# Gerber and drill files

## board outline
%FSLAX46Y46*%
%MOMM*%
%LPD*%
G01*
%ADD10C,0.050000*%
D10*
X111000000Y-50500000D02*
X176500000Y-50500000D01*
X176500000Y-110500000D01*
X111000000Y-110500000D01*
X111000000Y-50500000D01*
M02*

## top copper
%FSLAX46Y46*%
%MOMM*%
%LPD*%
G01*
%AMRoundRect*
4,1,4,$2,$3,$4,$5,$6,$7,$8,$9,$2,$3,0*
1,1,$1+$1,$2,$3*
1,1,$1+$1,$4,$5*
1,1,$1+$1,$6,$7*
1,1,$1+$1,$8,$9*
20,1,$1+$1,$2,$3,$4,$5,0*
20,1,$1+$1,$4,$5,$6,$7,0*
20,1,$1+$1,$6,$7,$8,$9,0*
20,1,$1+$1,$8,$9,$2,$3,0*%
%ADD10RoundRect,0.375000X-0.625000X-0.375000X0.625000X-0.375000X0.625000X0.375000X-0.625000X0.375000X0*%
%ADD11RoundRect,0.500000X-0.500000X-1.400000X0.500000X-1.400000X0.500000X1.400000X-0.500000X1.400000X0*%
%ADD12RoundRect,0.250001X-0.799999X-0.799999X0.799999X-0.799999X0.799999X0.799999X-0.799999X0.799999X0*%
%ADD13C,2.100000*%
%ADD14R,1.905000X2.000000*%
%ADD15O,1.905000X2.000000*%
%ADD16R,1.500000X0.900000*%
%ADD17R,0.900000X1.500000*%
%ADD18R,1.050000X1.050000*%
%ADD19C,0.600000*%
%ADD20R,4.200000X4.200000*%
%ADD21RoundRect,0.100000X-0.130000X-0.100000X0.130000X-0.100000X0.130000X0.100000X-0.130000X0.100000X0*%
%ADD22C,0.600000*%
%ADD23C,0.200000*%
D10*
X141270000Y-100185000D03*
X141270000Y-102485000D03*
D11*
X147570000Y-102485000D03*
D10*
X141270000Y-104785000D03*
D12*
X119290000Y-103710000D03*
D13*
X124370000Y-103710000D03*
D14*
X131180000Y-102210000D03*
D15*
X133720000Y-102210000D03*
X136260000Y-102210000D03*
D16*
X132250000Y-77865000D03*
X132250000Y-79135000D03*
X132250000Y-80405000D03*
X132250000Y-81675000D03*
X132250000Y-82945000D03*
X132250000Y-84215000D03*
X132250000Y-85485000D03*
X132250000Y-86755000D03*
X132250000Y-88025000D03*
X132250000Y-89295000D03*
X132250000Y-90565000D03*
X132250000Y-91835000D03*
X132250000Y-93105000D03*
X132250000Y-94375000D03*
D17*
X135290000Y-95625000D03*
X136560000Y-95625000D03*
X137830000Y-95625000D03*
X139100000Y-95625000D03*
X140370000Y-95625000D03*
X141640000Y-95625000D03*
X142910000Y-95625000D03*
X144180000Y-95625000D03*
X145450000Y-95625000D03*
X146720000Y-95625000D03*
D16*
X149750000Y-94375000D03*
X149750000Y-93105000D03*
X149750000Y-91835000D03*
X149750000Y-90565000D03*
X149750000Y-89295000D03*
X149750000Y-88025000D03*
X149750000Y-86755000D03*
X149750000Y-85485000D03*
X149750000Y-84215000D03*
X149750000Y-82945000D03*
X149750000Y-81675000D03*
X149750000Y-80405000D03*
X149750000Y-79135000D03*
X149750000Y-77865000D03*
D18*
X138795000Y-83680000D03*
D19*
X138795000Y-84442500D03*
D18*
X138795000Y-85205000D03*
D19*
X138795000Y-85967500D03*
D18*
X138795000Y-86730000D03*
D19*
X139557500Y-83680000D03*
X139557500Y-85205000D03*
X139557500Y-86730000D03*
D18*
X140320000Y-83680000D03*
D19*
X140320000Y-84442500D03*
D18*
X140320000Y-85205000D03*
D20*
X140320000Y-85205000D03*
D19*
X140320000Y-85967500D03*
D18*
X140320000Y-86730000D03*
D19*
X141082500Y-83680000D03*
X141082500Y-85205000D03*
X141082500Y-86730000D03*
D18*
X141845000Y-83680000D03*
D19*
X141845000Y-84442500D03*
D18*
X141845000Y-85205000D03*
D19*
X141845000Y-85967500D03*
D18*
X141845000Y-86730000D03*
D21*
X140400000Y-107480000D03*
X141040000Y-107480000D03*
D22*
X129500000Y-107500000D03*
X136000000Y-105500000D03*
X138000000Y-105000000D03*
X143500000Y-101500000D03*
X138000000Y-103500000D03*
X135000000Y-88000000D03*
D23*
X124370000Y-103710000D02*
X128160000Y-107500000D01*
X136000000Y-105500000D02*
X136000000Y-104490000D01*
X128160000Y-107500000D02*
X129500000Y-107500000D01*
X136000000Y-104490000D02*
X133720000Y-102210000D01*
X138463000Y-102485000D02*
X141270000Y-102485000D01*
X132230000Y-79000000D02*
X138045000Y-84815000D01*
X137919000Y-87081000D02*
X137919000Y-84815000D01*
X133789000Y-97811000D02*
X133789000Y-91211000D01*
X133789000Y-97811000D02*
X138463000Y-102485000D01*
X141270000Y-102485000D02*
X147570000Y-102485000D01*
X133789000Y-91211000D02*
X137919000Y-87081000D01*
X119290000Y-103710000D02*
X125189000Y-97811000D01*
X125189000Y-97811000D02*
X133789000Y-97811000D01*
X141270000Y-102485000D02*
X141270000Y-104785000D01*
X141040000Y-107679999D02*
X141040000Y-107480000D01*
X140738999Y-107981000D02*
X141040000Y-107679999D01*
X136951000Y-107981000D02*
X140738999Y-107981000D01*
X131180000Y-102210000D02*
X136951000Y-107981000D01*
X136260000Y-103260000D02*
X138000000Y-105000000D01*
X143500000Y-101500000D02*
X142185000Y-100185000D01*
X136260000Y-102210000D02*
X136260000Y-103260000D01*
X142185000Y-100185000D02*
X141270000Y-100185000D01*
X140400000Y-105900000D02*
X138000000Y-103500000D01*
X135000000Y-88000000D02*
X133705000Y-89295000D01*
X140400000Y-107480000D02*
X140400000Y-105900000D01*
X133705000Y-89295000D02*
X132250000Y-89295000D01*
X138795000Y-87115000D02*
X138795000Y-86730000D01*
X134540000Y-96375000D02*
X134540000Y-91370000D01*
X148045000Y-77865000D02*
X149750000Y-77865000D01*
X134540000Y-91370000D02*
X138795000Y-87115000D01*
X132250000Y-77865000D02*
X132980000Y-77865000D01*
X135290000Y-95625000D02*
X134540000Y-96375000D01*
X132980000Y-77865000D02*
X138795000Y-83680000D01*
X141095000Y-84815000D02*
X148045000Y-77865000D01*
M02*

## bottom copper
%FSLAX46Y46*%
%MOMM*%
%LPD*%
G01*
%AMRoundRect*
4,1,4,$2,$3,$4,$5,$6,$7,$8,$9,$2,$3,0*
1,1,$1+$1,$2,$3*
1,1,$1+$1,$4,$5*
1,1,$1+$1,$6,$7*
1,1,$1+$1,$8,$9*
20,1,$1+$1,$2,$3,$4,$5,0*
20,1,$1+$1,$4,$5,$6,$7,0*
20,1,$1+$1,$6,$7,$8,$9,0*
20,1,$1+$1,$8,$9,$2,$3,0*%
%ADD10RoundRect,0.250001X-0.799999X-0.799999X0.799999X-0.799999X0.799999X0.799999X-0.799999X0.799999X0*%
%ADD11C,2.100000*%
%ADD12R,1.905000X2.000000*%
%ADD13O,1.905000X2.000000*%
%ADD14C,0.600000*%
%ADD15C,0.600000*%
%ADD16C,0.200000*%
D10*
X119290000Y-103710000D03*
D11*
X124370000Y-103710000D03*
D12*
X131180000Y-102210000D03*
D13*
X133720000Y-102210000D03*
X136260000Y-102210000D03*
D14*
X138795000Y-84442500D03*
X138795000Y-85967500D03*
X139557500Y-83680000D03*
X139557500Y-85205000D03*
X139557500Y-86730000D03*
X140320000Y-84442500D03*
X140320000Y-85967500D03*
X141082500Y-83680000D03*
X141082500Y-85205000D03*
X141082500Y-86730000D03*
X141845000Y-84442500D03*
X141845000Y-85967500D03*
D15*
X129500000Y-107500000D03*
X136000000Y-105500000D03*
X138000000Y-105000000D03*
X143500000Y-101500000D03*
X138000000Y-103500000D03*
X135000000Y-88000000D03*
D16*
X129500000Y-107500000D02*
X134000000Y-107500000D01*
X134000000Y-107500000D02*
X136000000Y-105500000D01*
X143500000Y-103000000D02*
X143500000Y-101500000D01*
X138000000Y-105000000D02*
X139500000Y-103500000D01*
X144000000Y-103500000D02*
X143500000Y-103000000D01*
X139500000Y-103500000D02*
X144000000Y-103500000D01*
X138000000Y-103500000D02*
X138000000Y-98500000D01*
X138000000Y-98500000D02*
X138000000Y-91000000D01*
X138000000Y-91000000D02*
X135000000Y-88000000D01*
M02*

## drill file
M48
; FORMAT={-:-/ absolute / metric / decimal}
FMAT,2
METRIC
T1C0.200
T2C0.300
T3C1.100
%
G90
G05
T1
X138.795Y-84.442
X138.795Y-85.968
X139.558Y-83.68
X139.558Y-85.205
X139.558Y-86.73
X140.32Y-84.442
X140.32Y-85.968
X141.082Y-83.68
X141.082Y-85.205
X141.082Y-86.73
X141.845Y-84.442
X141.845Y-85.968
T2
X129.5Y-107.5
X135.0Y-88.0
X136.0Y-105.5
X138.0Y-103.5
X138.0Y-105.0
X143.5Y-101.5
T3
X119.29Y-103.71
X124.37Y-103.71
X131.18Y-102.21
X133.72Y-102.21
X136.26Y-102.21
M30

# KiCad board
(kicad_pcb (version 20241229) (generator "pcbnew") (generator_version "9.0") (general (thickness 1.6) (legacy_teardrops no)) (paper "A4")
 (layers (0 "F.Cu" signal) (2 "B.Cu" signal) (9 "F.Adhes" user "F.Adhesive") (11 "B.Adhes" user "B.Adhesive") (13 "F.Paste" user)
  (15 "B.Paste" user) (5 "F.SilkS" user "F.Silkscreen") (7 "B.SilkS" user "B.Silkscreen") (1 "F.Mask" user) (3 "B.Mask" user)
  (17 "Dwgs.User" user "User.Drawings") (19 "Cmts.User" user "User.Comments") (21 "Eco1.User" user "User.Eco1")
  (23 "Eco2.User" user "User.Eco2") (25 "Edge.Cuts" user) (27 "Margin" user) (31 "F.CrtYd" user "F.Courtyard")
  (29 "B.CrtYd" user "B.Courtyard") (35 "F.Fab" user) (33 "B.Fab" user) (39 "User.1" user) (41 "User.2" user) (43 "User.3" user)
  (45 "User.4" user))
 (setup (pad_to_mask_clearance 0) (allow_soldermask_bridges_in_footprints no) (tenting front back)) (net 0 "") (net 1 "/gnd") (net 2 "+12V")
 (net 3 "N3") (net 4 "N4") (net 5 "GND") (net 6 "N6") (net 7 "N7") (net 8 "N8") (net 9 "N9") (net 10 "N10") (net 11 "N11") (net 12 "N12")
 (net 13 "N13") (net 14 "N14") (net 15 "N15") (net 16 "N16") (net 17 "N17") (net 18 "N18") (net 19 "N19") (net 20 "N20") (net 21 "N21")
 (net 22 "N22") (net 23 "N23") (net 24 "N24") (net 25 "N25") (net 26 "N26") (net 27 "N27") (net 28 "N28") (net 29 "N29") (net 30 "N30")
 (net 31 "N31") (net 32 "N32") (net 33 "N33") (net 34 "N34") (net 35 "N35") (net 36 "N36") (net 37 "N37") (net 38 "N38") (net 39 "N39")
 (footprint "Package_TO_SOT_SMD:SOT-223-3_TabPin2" (layer "F.Cu") (at 144.42 102.485)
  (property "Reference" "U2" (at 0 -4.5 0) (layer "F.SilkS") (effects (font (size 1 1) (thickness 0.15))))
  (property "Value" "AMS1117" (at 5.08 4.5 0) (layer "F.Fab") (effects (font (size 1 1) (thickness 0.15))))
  (pad "1" smd roundrect (at -3.15 -2.3) (size 2 1.5) (layers "F.Cu" "F.Mask" "F.Paste") (roundrect_rratio 0.25) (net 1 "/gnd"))
  (pad "2" smd roundrect (at -3.15 0) (size 2 1.5) (layers "F.Cu" "F.Mask" "F.Paste") (roundrect_rratio 0.25) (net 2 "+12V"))
  (pad "2" smd roundrect (at 3.15 0) (size 2 3.8) (layers "F.Cu" "F.Mask" "F.Paste") (roundrect_rratio 0.25) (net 2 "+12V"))
  (pad "3" smd roundrect (at -3.15 2.3) (size 2 1.5) (layers "F.Cu" "F.Mask" "F.Paste") (roundrect_rratio 0.25) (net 2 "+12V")))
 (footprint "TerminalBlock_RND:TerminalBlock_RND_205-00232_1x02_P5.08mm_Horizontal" (layer "F.Cu") (at 119.29 103.71)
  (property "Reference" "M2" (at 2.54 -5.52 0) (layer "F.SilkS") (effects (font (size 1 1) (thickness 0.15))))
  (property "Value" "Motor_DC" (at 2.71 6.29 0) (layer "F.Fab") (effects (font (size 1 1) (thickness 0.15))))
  (pad "1" thru_hole roundrect (at 0 0) (size 2.1 2.1) (drill 1.1) (layers "*.Cu" "*.Mask") (remove_unused_layers no)
   (roundrect_rratio 0.119048) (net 2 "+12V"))
  (pad "2" thru_hole circle (at 5.08 0) (size 2.1 2.1) (drill 1.1) (layers "*.Cu" "*.Mask") (remove_unused_layers no) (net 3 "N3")))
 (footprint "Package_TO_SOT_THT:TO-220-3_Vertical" (layer "F.Cu") (at 131.18 102.21)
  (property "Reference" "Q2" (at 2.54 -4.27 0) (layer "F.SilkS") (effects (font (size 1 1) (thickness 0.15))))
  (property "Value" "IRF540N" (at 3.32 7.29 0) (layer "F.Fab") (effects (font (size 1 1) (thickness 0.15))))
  (pad "1" thru_hole rect (at 0 0) (size 1.905 2) (drill 1.1) (layers "*.Cu" "*.Mask") (remove_unused_layers no) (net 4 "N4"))
  (pad "2" thru_hole oval (at 2.54 0) (size 1.905 2) (drill 1.1) (layers "*.Cu" "*.Mask") (remove_unused_layers no) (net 3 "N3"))
  (pad "3" thru_hole oval (at 5.08 0) (size 1.905 2) (drill 1.1) (layers "*.Cu" "*.Mask") (remove_unused_layers no) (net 1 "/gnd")))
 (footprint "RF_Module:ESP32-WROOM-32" (layer "F.Cu") (at 141 86.115)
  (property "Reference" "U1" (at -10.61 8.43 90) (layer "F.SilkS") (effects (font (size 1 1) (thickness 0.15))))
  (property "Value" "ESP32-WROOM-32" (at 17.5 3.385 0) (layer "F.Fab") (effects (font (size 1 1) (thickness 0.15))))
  (pad "1" smd rect (at -8.75 -8.25) (size 1.5 0.9) (layers "F.Cu" "F.Mask" "F.Paste") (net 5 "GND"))
  (pad "2" smd rect (at -8.75 -6.98) (size 1.5 0.9) (layers "F.Cu" "F.Mask" "F.Paste") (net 2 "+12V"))
  (pad "3" smd rect (at -8.75 -5.71) (size 1.5 0.9) (layers "F.Cu" "F.Mask" "F.Paste") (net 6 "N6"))
  (pad "4" smd rect (at -8.75 -4.44) (size 1.5 0.9) (layers "F.Cu" "F.Mask" "F.Paste") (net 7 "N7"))
  (pad "5" smd rect (at -8.75 -3.17) (size 1.5 0.9) (layers "F.Cu" "F.Mask" "F.Paste") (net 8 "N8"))
  (pad "6" smd rect (at -8.75 -1.9) (size 1.5 0.9) (layers "F.Cu" "F.Mask" "F.Paste") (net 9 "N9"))
  (pad "7" smd rect (at -8.75 -0.63) (size 1.5 0.9) (layers "F.Cu" "F.Mask" "F.Paste") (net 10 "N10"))
  (pad "8" smd rect (at -8.75 0.64) (size 1.5 0.9) (layers "F.Cu" "F.Mask" "F.Paste") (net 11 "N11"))
  (pad "9" smd rect (at -8.75 1.91) (size 1.5 0.9) (layers "F.Cu" "F.Mask" "F.Paste") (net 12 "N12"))
  (pad "10" smd rect (at -8.75 3.18) (size 1.5 0.9) (layers "F.Cu" "F.Mask" "F.Paste") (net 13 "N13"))
  (pad "11" smd rect (at -8.75 4.45) (size 1.5 0.9) (layers "F.Cu" "F.Mask" "F.Paste") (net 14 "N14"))
  (pad "12" smd rect (at -8.75 5.72) (size 1.5 0.9) (layers "F.Cu" "F.Mask" "F.Paste") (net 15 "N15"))
  (pad "13" smd rect (at -8.75 6.99) (size 1.5 0.9) (layers "F.Cu" "F.Mask" "F.Paste") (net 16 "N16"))
  (pad "14" smd rect (at -8.75 8.26) (size 1.5 0.9) (layers "F.Cu" "F.Mask" "F.Paste") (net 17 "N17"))
  (pad "15" smd rect (at -5.71 9.51 90) (size 1.5 0.9) (layers "F.Cu" "F.Mask" "F.Paste") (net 5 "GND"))
  (pad "16" smd rect (at -4.44 9.51 90) (size 1.5 0.9) (layers "F.Cu" "F.Mask" "F.Paste") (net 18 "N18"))
  (pad "17" smd rect (at -3.17 9.51 90) (size 1.5 0.9) (layers "F.Cu" "F.Mask" "F.Paste") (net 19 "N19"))
  (pad "18" smd rect (at -1.9 9.51 90) (size 1.5 0.9) (layers "F.Cu" "F.Mask" "F.Paste") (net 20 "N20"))
  (pad "19" smd rect (at -0.63 9.51 90) (size 1.5 0.9) (layers "F.Cu" "F.Mask" "F.Paste") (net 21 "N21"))
  (pad "20" smd rect (at 0.64 9.51 90) (size 1.5 0.9) (layers "F.Cu" "F.Mask" "F.Paste") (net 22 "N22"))
  (pad "21" smd rect (at 1.91 9.51 90) (size 1.5 0.9) (layers "F.Cu" "F.Mask" "F.Paste") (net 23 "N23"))
  (pad "22" smd rect (at 3.18 9.51 90) (size 1.5 0.9) (layers "F.Cu" "F.Mask" "F.Paste") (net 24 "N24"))
  (pad "23" smd rect (at 4.45 9.51 90) (size 1.5 0.9) (layers "F.Cu" "F.Mask" "F.Paste") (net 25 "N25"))
  (pad "24" smd rect (at 5.72 9.51 90) (size 1.5 0.9) (layers "F.Cu" "F.Mask" "F.Paste") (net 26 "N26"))
  (pad "25" smd rect (at 8.75 8.26) (size 1.5 0.9) (layers "F.Cu" "F.Mask" "F.Paste") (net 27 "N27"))
  (pad "26" smd rect (at 8.75 6.99) (size 1.5 0.9) (layers "F.Cu" "F.Mask" "F.Paste") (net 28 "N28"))
  (pad "27" smd rect (at 8.75 5.72) (size 1.5 0.9) (layers "F.Cu" "F.Mask" "F.Paste") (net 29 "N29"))
  (pad "28" smd rect (at 8.75 4.45) (size 1.5 0.9) (layers "F.Cu" "F.Mask" "F.Paste") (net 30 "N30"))
  (pad "29" smd rect (at 8.75 3.18) (size 1.5 0.9) (layers "F.Cu" "F.Mask" "F.Paste") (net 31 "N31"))
  (pad "30" smd rect (at 8.75 1.91) (size 1.5 0.9) (layers "F.Cu" "F.Mask" "F.Paste") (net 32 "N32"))
  (pad "31" smd rect (at 8.75 0.64) (size 1.5 0.9) (layers "F.Cu" "F.Mask" "F.Paste") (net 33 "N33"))
  (pad "32" smd rect (at 8.75 -0.63) (size 1.5 0.9) (layers "F.Cu" "F.Mask" "F.Paste") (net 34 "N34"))
  (pad "33" smd rect (at 8.75 -1.9) (size 1.5 0.9) (layers "F.Cu" "F.Mask" "F.Paste") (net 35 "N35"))
  (pad "34" smd rect (at 8.75 -3.17) (size 1.5 0.9) (layers "F.Cu" "F.Mask" "F.Paste") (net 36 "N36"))
  (pad "35" smd rect (at 8.75 -4.44) (size 1.5 0.9) (layers "F.Cu" "F.Mask" "F.Paste") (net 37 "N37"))
  (pad "36" smd rect (at 8.75 -5.71) (size 1.5 0.9) (layers "F.Cu" "F.Mask" "F.Paste") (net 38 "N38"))
  (pad "37" smd rect (at 8.75 -6.98) (size 1.5 0.9) (layers "F.Cu" "F.Mask" "F.Paste") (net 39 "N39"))
  (pad "38" smd rect (at 8.75 -8.25) (size 1.5 0.9) (layers "F.Cu" "F.Mask" "F.Paste") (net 5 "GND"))
  (pad "39" smd rect (at -2.205 -2.435) (size 1.05 1.05) (layers "F.Cu" "F.Paste") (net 5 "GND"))
  (pad "39" thru_hole circle (at -2.205 -1.6725) (size 0.6 0.6) (drill 0.2) (layers "*.Cu" "F.Mask") (remove_unused_layers no) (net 5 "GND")
   (zone_connect 2))
  (pad "39" smd rect (at -2.205 -0.91) (size 1.05 1.05) (layers "F.Cu" "F.Paste") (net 5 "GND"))
  (pad "39" thru_hole circle (at -2.205 -0.1475) (size 0.6 0.6) (drill 0.2) (layers "*.Cu" "F.Mask") (remove_unused_layers no) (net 5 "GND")
   (zone_connect 2))
  (pad "39" smd rect (at -2.205 0.615) (size 1.05 1.05) (layers "F.Cu" "F.Paste") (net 5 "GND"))
  (pad "39" thru_hole circle (at -1.4425 -2.435) (size 0.6 0.6) (drill 0.2) (layers "*.Cu" "F.Mask") (remove_unused_layers no) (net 5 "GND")
   (zone_connect 2))
  (pad "39" thru_hole circle (at -1.4425 -0.91) (size 0.6 0.6) (drill 0.2) (layers "*.Cu" "F.Mask") (remove_unused_layers no) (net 5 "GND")
   (zone_connect 2))
  (pad "39" thru_hole circle (at -1.4425 0.615) (size 0.6 0.6) (drill 0.2) (layers "*.Cu" "F.Mask") (remove_unused_layers no) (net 5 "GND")
   (zone_connect 2))
  (pad "39" smd rect (at -0.68 -2.435) (size 1.05 1.05) (layers "F.Cu" "F.Paste") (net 5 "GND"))
  (pad "39" thru_hole circle (at -0.68 -1.6725) (size 0.6 0.6) (drill 0.2) (layers "*.Cu" "F.Mask") (remove_unused_layers no) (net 5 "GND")
   (zone_connect 2))
  (pad "39" smd rect (at -0.68 -0.91) (size 1.05 1.05) (layers "F.Cu" "F.Paste") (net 5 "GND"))
  (pad "39" smd rect (at -0.68 -0.91) (size 4.2 4.2) (layers "F.Cu" "F.Mask") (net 5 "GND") (zone_connect 2))
  (pad "39" thru_hole circle (at -0.68 -0.1475) (size 0.6 0.6) (drill 0.2) (layers "*.Cu" "F.Mask") (remove_unused_layers no) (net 5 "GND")
   (zone_connect 2))
  (pad "39" smd rect (at -0.68 0.615) (size 1.05 1.05) (layers "F.Cu" "F.Paste") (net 5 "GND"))
  (pad "39" thru_hole circle (at 0.0825 -2.435) (size 0.6 0.6) (drill 0.2) (layers "*.Cu" "F.Mask") (remove_unused_layers no) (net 5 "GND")
   (zone_connect 2))
  (pad "39" thru_hole circle (at 0.0825 -0.91) (size 0.6 0.6) (drill 0.2) (layers "*.Cu" "F.Mask") (remove_unused_layers no) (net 5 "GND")
   (zone_connect 2))
  (pad "39" thru_hole circle (at 0.0825 0.615) (size 0.6 0.6) (drill 0.2) (layers "*.Cu" "F.Mask") (remove_unused_layers no) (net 5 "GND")
   (zone_connect 2))
  (pad "39" smd rect (at 0.845 -2.435) (size 1.05 1.05) (layers "F.Cu" "F.Paste") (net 5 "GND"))
  (pad "39" thru_hole circle (at 0.845 -1.6725) (size 0.6 0.6) (drill 0.2) (layers "*.Cu" "F.Mask") (remove_unused_layers no) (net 5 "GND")
   (zone_connect 2))
  (pad "39" smd rect (at 0.845 -0.91) (size 1.05 1.05) (layers "F.Cu" "F.Paste") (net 5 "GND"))
  (pad "39" thru_hole circle (at 0.845 -0.1475) (size 0.6 0.6) (drill 0.2) (layers "*.Cu" "F.Mask") (remove_unused_layers no) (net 5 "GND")
   (zone_connect 2))
  (pad "39" smd rect (at 0.845 0.615) (size 1.05 1.05) (layers "F.Cu" "F.Paste") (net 5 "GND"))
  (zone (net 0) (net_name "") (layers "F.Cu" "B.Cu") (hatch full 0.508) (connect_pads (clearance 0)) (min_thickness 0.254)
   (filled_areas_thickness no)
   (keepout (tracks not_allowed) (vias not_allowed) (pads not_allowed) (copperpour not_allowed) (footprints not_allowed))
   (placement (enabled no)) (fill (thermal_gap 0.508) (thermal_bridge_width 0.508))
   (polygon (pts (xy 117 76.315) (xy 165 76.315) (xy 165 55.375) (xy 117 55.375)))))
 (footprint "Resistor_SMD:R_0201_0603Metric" (layer "F.Cu") (at 140.72 107.48)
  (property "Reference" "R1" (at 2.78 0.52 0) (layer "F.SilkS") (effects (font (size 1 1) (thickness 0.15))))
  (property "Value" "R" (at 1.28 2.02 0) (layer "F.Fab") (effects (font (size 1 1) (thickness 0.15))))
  (pad "" smd roundrect (at -0.345 0) (size 0.318 0.36) (layers "F.Paste") (roundrect_rratio 0.25))
  (pad "" smd roundrect (at 0.345 0) (size 0.318 0.36) (layers "F.Paste") (roundrect_rratio 0.25))
  (pad "1" smd roundrect (at -0.32 0) (size 0.46 0.4) (layers "F.Cu" "F.Mask") (roundrect_rratio 0.25) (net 13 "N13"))
  (pad "2" smd roundrect (at 0.32 0) (size 0.46 0.4) (layers "F.Cu" "F.Mask") (roundrect_rratio 0.25) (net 4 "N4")))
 (gr_rect (start 111 50.5) (end 176.5 110.5) (stroke (width 0.05) (type default)) (fill no) (layer "Edge.Cuts"))
 (segment (start 124.37 103.71) (end 128.16 107.5) (width 0.2) (layer "F.Cu") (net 3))
 (segment (start 136 105.5) (end 136 104.49) (width 0.2) (layer "F.Cu") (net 3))
 (segment (start 128.16 107.5) (end 129.5 107.5) (width 0.2) (layer "F.Cu") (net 3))
 (segment (start 136 104.49) (end 133.72 102.21) (width 0.2) (layer "F.Cu") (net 3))
 (via (at 129.5 107.5) (size 0.6) (drill 0.3) (layers "F.Cu" "B.Cu") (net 3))
 (via (at 136 105.5) (size 0.6) (drill 0.3) (layers "F.Cu" "B.Cu") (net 3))
 (segment (start 129.5 107.5) (end 134 107.5) (width 0.2) (layer "B.Cu") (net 3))
 (segment (start 134 107.5) (end 136 105.5) (width 0.2) (layer "B.Cu") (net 3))
 (segment (start 138.463 102.485) (end 141.27 102.485) (width 0.2) (layer "F.Cu") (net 2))
 (segment (start 132.23 79) (end 138.045 84.815) (width 0.2) (layer "F.Cu") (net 2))
 (segment (start 137.919 87.081) (end 137.919 84.815) (width 0.2) (layer "F.Cu") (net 2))
 (segment (start 133.789 97.811) (end 133.789 91.211) (width 0.2) (layer "F.Cu") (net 2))
 (segment (start 133.789 97.811) (end 138.463 102.485) (width 0.2) (layer "F.Cu") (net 2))
 (segment (start 141.27 102.485) (end 147.57 102.485) (width 0.2) (layer "F.Cu") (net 2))
 (segment (start 133.789 91.211) (end 137.919 87.081) (width 0.2) (layer "F.Cu") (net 2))
 (segment (start 119.29 103.71) (end 125.189 97.811) (width 0.2) (layer "F.Cu") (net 2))
 (segment (start 125.189 97.811) (end 133.789 97.811) (width 0.2) (layer "F.Cu") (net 2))
 (segment (start 141.27 102.485) (end 141.27 104.785) (width 0.2) (layer "F.Cu") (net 2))
 (segment (start 141.04 107.679999) (end 141.04 107.48) (width 0.2) (layer "F.Cu") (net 4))
 (segment (start 140.738999 107.981) (end 141.04 107.679999) (width 0.2) (layer "F.Cu") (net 4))
 (segment (start 136.951 107.981) (end 140.738999 107.981) (width 0.2) (layer "F.Cu") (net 4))
 (segment (start 131.18 102.21) (end 136.951 107.981) (width 0.2) (layer "F.Cu") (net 4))
 (segment (start 136.26 103.26) (end 138 105) (width 0.2) (layer "F.Cu") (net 1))
 (segment (start 143.5 101.5) (end 142.185 100.185) (width 0.2) (layer "F.Cu") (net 1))
 (segment (start 136.26 102.21) (end 136.26 103.26) (width 0.2) (layer "F.Cu") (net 1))
 (segment (start 142.185 100.185) (end 141.27 100.185) (width 0.2) (layer "F.Cu") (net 1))
 (via (at 138 105) (size 0.6) (drill 0.3) (layers "F.Cu" "B.Cu") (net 1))
 (via (at 143.5 101.5) (size 0.6) (drill 0.3) (layers "F.Cu" "B.Cu") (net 1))
 (segment (start 143.5 103) (end 143.5 101.5) (width 0.2) (layer "B.Cu") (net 1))
 (segment (start 138 105) (end 139.5 103.5) (width 0.2) (layer "B.Cu") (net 1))
 (segment (start 144 103.5) (end 143.5 103) (width 0.2) (layer "B.Cu") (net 1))
 (segment (start 139.5 103.5) (end 144 103.5) (width 0.2) (layer "B.Cu") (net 1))
 (segment (start 140.4 105.9) (end 138 103.5) (width 0.2) (layer "F.Cu") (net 13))
 (segment (start 135 88) (end 133.705 89.295) (width 0.2) (layer "F.Cu") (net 13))
 (segment (start 140.4 107.48) (end 140.4 105.9) (width 0.2) (layer "F.Cu") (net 13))
 (segment (start 133.705 89.295) (end 132.25 89.295) (width 0.2) (layer "F.Cu") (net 13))
 (via (at 138 103.5) (size 0.6) (drill 0.3) (layers "F.Cu" "B.Cu") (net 13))
 (via (at 135 88) (size 0.6) (drill 0.3) (layers "F.Cu" "B.Cu") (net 13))
 (segment (start 138 103.5) (end 138 98.5) (width 0.2) (layer "B.Cu") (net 13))
 (segment (start 138 98.5) (end 138 91) (width 0.2) (layer "B.Cu") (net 13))
 (segment (start 138 91) (end 135 88) (width 0.2) (layer "B.Cu") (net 13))
 (segment (start 138.795 87.115) (end 138.795 86.73) (width 0.2) (layer "F.Cu") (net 5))
 (segment (start 134.54 96.375) (end 134.54 91.37) (width 0.2) (layer "F.Cu") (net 5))
 (segment (start 148.045 77.865) (end 149.75 77.865) (width 0.2) (layer "F.Cu") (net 5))
 (segment (start 134.54 91.37) (end 138.795 87.115) (width 0.2) (layer "F.Cu") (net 5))
 (segment (start 132.25 77.865) (end 132.98 77.865) (width 0.2) (layer "F.Cu") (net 5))
 (segment (start 135.29 95.625) (end 134.54 96.375) (width 0.2) (layer "F.Cu") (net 5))
 (segment (start 132.98 77.865) (end 138.795 83.68) (width 0.2) (layer "F.Cu") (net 5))
 (segment (start 141.095 84.815) (end 148.045 77.865) (width 0.2) (layer "F.Cu") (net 5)))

